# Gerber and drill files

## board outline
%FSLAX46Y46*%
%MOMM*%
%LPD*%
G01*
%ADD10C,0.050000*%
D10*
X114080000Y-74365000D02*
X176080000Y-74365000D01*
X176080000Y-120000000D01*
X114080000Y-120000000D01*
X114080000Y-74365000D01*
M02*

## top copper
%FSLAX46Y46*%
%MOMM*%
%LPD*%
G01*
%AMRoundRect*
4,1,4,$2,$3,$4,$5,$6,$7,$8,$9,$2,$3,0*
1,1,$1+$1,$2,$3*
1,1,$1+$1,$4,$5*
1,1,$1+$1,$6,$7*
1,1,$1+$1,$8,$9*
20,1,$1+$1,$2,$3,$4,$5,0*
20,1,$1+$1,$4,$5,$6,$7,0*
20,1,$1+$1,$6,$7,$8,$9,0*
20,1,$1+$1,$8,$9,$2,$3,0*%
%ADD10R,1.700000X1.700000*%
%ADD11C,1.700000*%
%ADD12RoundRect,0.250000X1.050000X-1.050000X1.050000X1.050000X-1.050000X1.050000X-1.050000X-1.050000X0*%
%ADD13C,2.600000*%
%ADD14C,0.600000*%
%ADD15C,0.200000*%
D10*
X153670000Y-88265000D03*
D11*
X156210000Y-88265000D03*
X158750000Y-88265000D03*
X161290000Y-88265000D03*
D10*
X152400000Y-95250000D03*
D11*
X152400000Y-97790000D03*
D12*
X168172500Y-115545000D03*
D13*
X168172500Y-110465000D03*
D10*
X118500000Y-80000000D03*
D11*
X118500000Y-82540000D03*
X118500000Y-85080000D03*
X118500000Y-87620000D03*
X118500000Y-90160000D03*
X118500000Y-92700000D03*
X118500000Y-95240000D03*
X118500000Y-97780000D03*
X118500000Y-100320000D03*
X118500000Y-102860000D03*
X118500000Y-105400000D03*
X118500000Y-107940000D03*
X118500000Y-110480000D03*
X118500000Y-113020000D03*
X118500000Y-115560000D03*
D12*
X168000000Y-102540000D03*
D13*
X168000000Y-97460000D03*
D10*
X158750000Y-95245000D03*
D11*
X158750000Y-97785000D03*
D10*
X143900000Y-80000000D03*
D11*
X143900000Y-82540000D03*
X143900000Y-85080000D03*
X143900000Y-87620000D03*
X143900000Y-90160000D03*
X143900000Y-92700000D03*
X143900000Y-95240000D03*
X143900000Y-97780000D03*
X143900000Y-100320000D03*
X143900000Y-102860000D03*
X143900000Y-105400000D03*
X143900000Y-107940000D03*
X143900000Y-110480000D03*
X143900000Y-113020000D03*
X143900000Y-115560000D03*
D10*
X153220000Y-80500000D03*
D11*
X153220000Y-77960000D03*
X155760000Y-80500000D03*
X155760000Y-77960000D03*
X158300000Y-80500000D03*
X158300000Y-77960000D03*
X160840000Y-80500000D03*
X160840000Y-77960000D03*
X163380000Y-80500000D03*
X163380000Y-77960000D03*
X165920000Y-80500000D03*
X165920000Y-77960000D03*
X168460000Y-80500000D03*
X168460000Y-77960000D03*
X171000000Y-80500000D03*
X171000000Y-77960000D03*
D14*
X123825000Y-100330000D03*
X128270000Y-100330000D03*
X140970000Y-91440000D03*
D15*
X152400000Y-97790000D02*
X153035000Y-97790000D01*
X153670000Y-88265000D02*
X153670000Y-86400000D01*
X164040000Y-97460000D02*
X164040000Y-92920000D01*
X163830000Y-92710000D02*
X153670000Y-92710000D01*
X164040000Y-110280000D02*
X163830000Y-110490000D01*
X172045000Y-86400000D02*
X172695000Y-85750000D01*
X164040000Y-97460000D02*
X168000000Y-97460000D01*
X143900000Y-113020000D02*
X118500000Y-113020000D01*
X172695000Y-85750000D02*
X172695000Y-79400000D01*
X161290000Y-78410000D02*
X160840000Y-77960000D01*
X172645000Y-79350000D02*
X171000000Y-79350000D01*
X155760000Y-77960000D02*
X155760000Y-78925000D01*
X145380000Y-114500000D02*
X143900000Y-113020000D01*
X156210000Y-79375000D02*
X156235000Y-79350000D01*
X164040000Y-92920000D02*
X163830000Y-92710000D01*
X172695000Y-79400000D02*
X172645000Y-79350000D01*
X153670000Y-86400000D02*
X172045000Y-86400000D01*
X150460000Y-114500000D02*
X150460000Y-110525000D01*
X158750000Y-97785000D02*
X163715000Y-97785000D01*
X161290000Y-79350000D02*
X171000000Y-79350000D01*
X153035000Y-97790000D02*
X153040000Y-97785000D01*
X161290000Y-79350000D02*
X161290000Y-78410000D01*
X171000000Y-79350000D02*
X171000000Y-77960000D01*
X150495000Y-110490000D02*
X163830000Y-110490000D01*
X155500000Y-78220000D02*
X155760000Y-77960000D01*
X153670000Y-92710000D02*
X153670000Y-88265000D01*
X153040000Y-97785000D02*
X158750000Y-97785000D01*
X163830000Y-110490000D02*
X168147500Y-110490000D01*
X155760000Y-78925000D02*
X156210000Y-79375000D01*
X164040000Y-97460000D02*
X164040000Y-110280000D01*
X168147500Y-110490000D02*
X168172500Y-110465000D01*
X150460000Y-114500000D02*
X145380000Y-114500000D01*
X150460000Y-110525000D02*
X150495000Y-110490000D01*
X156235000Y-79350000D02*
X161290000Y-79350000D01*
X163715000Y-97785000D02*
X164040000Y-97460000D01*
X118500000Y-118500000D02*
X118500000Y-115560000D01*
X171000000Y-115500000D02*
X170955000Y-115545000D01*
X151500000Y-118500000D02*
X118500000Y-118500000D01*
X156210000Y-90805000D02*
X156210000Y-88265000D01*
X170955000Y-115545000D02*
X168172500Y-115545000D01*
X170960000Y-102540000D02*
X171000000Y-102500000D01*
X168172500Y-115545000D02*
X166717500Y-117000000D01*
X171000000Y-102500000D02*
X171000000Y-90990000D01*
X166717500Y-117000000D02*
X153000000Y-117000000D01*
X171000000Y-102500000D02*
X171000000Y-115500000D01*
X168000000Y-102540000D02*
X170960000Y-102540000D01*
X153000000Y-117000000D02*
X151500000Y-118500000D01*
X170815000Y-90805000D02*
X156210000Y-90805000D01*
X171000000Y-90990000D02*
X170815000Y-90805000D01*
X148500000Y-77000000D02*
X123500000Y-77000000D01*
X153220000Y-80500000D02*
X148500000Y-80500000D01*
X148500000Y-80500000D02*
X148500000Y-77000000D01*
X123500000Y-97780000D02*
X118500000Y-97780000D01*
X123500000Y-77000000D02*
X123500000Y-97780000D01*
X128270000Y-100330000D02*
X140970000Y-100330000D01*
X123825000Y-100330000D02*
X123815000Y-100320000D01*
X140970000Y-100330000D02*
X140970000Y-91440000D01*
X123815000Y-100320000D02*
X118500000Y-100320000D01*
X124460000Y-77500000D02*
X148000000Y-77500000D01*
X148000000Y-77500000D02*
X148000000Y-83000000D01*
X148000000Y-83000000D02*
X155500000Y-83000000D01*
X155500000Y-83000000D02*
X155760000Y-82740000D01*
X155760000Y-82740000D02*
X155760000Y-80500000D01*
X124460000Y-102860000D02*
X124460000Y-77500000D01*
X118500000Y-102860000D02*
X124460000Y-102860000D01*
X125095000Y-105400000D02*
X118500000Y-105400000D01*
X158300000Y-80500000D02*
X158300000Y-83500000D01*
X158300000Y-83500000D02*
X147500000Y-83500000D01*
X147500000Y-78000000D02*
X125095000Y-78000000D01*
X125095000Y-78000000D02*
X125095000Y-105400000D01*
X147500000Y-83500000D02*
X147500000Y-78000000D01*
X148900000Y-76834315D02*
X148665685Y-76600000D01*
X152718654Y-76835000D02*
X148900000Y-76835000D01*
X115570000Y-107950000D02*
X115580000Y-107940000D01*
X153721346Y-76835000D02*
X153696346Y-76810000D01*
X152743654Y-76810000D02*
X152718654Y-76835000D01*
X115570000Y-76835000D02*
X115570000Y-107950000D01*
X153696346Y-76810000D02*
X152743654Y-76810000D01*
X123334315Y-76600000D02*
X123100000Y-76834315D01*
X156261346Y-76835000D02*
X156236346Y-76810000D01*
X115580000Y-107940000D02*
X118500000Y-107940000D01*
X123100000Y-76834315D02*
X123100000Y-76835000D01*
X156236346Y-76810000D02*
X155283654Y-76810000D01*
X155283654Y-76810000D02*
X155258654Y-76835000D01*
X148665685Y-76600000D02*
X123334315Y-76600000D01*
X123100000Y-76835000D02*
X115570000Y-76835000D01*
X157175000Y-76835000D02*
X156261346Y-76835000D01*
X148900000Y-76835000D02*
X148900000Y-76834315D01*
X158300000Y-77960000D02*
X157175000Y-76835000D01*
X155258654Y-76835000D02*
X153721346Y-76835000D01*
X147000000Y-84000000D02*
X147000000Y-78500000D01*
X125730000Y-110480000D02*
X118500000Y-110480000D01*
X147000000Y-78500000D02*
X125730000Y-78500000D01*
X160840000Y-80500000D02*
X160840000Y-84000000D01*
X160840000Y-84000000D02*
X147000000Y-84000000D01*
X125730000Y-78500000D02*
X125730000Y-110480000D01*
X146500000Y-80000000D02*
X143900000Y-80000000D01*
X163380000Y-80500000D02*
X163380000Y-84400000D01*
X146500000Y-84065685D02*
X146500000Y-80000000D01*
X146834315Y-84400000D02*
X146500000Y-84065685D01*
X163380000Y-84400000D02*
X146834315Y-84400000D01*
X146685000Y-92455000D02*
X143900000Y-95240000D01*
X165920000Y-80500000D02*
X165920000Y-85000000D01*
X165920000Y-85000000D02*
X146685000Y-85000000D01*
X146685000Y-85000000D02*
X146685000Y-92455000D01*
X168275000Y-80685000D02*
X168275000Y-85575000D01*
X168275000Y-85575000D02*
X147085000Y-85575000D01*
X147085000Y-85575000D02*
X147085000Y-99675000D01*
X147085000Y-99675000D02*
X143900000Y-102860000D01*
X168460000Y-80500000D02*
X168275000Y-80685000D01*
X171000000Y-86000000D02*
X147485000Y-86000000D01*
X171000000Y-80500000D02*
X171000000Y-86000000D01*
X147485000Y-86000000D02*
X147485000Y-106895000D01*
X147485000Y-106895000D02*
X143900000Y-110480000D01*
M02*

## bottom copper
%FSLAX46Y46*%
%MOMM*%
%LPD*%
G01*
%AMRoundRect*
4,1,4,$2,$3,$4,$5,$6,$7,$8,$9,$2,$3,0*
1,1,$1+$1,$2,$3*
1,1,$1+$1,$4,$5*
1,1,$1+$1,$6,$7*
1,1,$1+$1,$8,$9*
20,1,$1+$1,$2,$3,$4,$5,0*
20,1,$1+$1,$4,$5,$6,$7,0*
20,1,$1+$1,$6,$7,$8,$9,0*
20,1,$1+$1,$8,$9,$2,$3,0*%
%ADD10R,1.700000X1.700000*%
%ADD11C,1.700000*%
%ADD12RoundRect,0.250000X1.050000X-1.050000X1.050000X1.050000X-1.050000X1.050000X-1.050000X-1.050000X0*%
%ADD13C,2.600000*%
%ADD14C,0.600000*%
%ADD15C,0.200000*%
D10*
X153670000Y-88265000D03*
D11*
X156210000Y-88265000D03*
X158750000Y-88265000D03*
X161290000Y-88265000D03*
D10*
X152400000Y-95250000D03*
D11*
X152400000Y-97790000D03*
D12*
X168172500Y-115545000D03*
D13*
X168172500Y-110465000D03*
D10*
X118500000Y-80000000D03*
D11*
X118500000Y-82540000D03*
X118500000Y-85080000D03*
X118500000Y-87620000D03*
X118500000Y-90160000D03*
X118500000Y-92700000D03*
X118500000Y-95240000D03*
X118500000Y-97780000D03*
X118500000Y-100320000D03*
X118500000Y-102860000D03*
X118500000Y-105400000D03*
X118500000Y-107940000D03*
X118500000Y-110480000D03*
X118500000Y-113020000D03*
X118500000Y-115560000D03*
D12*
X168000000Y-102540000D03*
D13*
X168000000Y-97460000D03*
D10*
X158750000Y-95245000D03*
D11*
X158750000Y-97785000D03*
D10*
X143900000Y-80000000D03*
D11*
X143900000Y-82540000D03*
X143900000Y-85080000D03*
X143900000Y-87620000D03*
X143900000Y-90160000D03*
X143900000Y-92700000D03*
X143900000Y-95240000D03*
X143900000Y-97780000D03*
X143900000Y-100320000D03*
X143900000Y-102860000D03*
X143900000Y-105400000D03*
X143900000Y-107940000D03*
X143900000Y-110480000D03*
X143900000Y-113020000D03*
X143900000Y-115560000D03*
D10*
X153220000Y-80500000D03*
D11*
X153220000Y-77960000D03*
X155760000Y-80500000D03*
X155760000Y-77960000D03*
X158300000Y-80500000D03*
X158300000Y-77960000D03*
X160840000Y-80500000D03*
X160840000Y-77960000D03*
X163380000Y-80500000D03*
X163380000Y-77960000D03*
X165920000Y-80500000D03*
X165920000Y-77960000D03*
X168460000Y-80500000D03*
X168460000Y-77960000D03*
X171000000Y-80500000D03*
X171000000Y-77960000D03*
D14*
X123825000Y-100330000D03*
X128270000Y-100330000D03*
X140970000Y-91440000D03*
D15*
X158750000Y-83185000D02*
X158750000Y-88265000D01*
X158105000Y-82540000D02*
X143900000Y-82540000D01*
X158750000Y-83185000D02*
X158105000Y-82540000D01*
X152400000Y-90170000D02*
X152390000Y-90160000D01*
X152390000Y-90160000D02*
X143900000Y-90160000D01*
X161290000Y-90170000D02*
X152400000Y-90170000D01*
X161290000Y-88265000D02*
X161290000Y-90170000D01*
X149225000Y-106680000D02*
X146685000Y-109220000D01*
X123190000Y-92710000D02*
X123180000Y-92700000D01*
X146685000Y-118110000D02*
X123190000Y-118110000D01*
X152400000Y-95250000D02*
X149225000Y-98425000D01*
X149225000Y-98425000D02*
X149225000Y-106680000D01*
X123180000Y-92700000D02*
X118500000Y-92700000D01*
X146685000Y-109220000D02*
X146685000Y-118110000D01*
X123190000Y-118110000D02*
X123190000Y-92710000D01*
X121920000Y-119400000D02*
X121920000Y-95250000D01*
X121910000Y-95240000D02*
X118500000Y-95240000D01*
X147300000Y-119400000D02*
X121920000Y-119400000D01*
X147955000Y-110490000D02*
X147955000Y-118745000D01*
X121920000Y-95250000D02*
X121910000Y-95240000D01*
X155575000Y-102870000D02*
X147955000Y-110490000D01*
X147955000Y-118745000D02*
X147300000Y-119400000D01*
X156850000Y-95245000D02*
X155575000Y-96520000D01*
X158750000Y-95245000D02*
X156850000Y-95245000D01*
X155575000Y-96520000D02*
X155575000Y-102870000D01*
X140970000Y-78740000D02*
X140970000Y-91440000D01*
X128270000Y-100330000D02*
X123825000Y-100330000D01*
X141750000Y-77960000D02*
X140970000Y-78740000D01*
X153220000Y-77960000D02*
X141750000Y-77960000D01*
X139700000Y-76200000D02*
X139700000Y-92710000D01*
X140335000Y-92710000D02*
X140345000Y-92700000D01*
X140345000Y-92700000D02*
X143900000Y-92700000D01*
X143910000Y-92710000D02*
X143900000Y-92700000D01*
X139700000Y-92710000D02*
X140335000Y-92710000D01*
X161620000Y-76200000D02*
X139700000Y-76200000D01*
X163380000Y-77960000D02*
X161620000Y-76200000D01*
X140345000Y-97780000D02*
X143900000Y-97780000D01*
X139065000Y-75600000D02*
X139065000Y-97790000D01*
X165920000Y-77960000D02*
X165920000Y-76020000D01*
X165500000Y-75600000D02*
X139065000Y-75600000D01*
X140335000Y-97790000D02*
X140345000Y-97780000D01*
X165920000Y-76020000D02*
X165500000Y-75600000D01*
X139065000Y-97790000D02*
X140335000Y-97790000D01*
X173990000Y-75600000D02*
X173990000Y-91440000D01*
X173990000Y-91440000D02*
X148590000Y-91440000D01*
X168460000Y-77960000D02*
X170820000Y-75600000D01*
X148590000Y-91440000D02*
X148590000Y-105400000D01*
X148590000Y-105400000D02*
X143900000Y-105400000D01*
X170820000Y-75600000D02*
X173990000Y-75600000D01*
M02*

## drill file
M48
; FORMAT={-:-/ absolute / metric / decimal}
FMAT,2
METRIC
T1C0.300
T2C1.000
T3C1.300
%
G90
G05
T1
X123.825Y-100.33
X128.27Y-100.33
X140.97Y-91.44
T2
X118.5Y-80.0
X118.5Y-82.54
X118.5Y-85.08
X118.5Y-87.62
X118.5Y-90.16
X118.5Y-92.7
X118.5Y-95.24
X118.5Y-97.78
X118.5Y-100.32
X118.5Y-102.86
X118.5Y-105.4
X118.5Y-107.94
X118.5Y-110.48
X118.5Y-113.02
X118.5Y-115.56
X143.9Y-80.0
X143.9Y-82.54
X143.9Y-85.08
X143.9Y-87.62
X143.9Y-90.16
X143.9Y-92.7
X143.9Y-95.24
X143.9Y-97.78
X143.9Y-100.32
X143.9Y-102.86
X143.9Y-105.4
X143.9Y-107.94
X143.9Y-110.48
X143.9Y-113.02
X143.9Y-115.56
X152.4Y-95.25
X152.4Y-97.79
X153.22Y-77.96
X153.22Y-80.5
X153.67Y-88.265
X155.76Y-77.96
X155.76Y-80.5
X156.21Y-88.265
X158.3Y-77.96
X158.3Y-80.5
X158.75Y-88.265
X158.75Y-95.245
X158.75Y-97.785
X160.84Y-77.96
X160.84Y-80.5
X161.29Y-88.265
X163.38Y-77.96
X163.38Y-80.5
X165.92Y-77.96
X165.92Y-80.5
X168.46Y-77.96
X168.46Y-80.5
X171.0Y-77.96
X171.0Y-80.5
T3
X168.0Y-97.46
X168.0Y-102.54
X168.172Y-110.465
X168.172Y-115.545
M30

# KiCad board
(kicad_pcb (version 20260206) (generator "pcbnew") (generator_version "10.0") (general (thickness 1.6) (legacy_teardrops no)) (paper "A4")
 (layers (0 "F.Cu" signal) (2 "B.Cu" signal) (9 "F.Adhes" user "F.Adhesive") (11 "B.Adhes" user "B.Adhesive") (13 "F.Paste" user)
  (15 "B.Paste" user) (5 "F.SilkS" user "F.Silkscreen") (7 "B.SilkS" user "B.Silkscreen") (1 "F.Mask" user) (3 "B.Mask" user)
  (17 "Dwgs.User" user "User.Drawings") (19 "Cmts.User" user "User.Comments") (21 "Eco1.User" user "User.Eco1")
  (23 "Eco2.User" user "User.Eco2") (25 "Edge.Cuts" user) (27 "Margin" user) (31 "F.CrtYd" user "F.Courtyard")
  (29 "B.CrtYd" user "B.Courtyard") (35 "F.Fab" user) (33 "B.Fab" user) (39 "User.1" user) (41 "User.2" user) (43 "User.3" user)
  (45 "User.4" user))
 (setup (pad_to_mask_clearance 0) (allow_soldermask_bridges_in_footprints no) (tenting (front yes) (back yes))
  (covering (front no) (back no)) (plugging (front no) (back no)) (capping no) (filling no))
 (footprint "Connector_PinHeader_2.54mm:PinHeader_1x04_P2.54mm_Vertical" (layer "F.Cu") (at 153.67 88.265 90)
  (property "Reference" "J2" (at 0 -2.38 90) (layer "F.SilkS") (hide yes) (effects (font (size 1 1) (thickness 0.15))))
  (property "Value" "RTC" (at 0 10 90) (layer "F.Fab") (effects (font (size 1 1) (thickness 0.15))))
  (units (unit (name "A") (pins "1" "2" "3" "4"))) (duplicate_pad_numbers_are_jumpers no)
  (pad "1" thru_hole rect (at 0 0 90) (size 1.7 1.7) (drill 1) (layers "*.Cu" "*.Mask") (remove_unused_layers no) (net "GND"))
  (pad "2" thru_hole circle (at 0 2.54 90) (size 1.7 1.7) (drill 1) (layers "*.Cu" "*.Mask") (remove_unused_layers no) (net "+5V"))
  (pad "3" thru_hole circle (at 0 5.08 90) (size 1.7 1.7) (drill 1) (layers "*.Cu" "*.Mask") (remove_unused_layers no) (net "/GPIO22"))
  (pad "4" thru_hole circle (at 0 7.62 90) (size 1.7 1.7) (drill 1) (layers "*.Cu" "*.Mask") (remove_unused_layers no) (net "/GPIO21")))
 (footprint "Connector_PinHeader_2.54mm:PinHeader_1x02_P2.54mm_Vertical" (layer "F.Cu") (at 152.4 95.25)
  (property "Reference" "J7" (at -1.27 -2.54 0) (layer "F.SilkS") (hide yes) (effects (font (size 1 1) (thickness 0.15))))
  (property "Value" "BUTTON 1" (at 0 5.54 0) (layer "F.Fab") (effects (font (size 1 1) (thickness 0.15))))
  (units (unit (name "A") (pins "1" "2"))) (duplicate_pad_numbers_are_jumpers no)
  (pad "1" thru_hole rect (at 0 0) (size 1.7 1.7) (drill 1) (layers "*.Cu" "*.Mask") (remove_unused_layers no) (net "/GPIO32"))
  (pad "2" thru_hole circle (at 0 2.54) (size 1.7 1.7) (drill 1) (layers "*.Cu" "*.Mask") (remove_unused_layers no) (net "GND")))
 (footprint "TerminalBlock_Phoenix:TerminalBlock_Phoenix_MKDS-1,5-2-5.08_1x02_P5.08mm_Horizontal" (layer "F.Cu") (at 168.1725 115.545 90)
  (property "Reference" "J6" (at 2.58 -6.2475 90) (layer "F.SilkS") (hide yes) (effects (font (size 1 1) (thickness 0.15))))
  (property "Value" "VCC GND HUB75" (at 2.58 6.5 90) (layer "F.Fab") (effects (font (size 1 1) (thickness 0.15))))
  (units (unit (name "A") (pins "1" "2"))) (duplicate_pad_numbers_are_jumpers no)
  (pad "1" thru_hole roundrect (at 0 0 90) (size 2.6 2.6) (drill 1.3) (layers "*.Cu" "*.Mask") (remove_unused_layers no)
   (roundrect_rratio 0.096154) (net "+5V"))
  (pad "2" thru_hole circle (at 5.08 0 90) (size 2.6 2.6) (drill 1.3) (layers "*.Cu" "*.Mask") (remove_unused_layers no) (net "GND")))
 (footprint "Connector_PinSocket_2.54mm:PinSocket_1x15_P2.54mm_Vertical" (layer "F.Cu") (at 118.5 80)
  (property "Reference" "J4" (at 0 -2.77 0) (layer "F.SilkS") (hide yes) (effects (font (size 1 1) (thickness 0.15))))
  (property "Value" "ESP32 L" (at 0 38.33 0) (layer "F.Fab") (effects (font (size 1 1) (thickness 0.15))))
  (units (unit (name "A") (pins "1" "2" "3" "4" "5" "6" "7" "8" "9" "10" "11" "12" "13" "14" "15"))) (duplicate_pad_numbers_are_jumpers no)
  (pad "1" thru_hole rect (at 0 0) (size 1.7 1.7) (drill 1) (layers "*.Cu" "*.Mask") (remove_unused_layers no)
   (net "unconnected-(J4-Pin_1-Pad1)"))
  (pad "2" thru_hole circle (at 0 2.54) (size 1.7 1.7) (drill 1) (layers "*.Cu" "*.Mask") (remove_unused_layers no)
   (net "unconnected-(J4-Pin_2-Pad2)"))
  (pad "3" thru_hole circle (at 0 5.08) (size 1.7 1.7) (drill 1) (layers "*.Cu" "*.Mask") (remove_unused_layers no)
   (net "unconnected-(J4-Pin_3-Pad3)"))
  (pad "4" thru_hole circle (at 0 7.62) (size 1.7 1.7) (drill 1) (layers "*.Cu" "*.Mask") (remove_unused_layers no)
   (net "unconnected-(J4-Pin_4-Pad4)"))
  (pad "5" thru_hole circle (at 0 10.16) (size 1.7 1.7) (drill 1) (layers "*.Cu" "*.Mask") (remove_unused_layers no)
   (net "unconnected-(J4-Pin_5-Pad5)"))
  (pad "6" thru_hole circle (at 0 12.7) (size 1.7 1.7) (drill 1) (layers "*.Cu" "*.Mask") (remove_unused_layers no) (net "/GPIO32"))
  (pad "7" thru_hole circle (at 0 15.24) (size 1.7 1.7) (drill 1) (layers "*.Cu" "*.Mask") (remove_unused_layers no) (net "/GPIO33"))
  (pad "8" thru_hole circle (at 0 17.78) (size 1.7 1.7) (drill 1) (layers "*.Cu" "*.Mask") (remove_unused_layers no) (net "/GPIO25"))
  (pad "9" thru_hole circle (at 0 20.32) (size 1.7 1.7) (drill 1) (layers "*.Cu" "*.Mask") (remove_unused_layers no) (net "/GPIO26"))
  (pad "10" thru_hole circle (at 0 22.86) (size 1.7 1.7) (drill 1) (layers "*.Cu" "*.Mask") (remove_unused_layers no) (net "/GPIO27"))
  (pad "11" thru_hole circle (at 0 25.4) (size 1.7 1.7) (drill 1) (layers "*.Cu" "*.Mask") (remove_unused_layers no) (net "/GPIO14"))
  (pad "12" thru_hole circle (at 0 27.94) (size 1.7 1.7) (drill 1) (layers "*.Cu" "*.Mask") (remove_unused_layers no) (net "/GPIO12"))
  (pad "13" thru_hole circle (at 0 30.48) (size 1.7 1.7) (drill 1) (layers "*.Cu" "*.Mask") (remove_unused_layers no) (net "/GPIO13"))
  (pad "14" thru_hole circle (at 0 33.02) (size 1.7 1.7) (drill 1) (layers "*.Cu" "*.Mask") (remove_unused_layers no) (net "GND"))
  (pad "15" thru_hole circle (at 0 35.56) (size 1.7 1.7) (drill 1) (layers "*.Cu" "*.Mask") (remove_unused_layers no) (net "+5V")))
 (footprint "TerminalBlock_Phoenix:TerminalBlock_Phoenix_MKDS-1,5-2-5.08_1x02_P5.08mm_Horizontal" (layer "F.Cu") (at 168 102.54 90)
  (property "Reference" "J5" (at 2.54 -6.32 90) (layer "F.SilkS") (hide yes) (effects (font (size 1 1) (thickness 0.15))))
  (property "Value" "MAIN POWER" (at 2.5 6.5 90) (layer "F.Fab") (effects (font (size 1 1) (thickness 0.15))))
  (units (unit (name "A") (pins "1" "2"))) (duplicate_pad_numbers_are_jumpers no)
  (pad "1" thru_hole roundrect (at 0 0 90) (size 2.6 2.6) (drill 1.3) (layers "*.Cu" "*.Mask") (remove_unused_layers no)
   (roundrect_rratio 0.096154) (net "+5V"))
  (pad "2" thru_hole circle (at 5.08 0 90) (size 2.6 2.6) (drill 1.3) (layers "*.Cu" "*.Mask") (remove_unused_layers no) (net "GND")))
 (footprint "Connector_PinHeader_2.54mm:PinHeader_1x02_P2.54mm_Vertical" (layer "F.Cu") (at 158.75 95.245)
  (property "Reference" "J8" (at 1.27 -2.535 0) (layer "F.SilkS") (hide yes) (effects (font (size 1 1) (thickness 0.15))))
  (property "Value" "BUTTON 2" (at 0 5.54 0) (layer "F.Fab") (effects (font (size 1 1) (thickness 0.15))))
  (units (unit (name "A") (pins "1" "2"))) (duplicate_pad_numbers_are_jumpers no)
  (pad "1" thru_hole rect (at 0 0) (size 1.7 1.7) (drill 1) (layers "*.Cu" "*.Mask") (remove_unused_layers no) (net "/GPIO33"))
  (pad "2" thru_hole circle (at 0 2.54) (size 1.7 1.7) (drill 1) (layers "*.Cu" "*.Mask") (remove_unused_layers no) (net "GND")))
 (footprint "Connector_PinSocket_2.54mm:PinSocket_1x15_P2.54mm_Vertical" (layer "F.Cu") (at 143.9 80)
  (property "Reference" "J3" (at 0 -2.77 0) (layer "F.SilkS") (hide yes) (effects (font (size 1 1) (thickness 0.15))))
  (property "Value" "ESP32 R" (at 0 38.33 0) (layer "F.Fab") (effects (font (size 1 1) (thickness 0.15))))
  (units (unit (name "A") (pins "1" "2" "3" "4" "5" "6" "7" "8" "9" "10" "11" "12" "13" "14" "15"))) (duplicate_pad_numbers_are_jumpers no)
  (pad "1" thru_hole rect (at 0 0) (size 1.7 1.7) (drill 1) (layers "*.Cu" "*.Mask") (remove_unused_layers no) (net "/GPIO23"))
  (pad "2" thru_hole circle (at 0 2.54) (size 1.7 1.7) (drill 1) (layers "*.Cu" "*.Mask") (remove_unused_layers no) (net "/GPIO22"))
  (pad "3" thru_hole circle (at 0 5.08) (size 1.7 1.7) (drill 1) (layers "*.Cu" "*.Mask") (remove_unused_layers no)
   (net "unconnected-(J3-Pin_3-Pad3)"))
  (pad "4" thru_hole circle (at 0 7.62) (size 1.7 1.7) (drill 1) (layers "*.Cu" "*.Mask") (remove_unused_layers no)
   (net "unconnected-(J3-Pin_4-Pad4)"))
  (pad "5" thru_hole circle (at 0 10.16) (size 1.7 1.7) (drill 1) (layers "*.Cu" "*.Mask") (remove_unused_layers no) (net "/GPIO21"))
  (pad "6" thru_hole circle (at 0 12.7) (size 1.7 1.7) (drill 1) (layers "*.Cu" "*.Mask") (remove_unused_layers no) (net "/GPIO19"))
  (pad "7" thru_hole circle (at 0 15.24) (size 1.7 1.7) (drill 1) (layers "*.Cu" "*.Mask") (remove_unused_layers no) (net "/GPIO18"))
  (pad "8" thru_hole circle (at 0 17.78) (size 1.7 1.7) (drill 1) (layers "*.Cu" "*.Mask") (remove_unused_layers no) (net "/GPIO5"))
  (pad "9" thru_hole circle (at 0 20.32) (size 1.7 1.7) (drill 1) (layers "*.Cu" "*.Mask") (remove_unused_layers no)
   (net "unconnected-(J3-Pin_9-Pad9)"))
  (pad "10" thru_hole circle (at 0 22.86) (size 1.7 1.7) (drill 1) (layers "*.Cu" "*.Mask") (remove_unused_layers no) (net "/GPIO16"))
  (pad "11" thru_hole circle (at 0 25.4) (size 1.7 1.7) (drill 1) (layers "*.Cu" "*.Mask") (remove_unused_layers no) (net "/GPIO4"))
  (pad "12" thru_hole circle (at 0 27.94) (size 1.7 1.7) (drill 1) (layers "*.Cu" "*.Mask") (remove_unused_layers no)
   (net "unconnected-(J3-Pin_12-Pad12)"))
  (pad "13" thru_hole circle (at 0 30.48) (size 1.7 1.7) (drill 1) (layers "*.Cu" "*.Mask") (remove_unused_layers no) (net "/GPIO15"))
  (pad "14" thru_hole circle (at 0 33.02) (size 1.7 1.7) (drill 1) (layers "*.Cu" "*.Mask") (remove_unused_layers no) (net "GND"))
  (pad "15" thru_hole circle (at 0 35.56) (size 1.7 1.7) (drill 1) (layers "*.Cu" "*.Mask") (remove_unused_layers no)
   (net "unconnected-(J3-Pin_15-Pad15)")))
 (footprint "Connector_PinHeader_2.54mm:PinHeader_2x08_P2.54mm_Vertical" (layer "F.Cu") (at 153.22 80.5 90)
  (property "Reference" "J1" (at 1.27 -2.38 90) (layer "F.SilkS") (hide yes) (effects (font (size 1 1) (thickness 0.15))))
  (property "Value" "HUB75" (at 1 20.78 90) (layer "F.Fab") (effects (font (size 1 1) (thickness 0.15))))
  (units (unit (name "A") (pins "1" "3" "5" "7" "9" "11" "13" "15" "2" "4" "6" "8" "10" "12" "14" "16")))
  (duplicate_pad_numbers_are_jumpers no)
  (pad "1" thru_hole rect (at 0 0 90) (size 1.7 1.7) (drill 1) (layers "*.Cu" "*.Mask") (remove_unused_layers no) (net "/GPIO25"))
  (pad "2" thru_hole circle (at 2.54 0 90) (size 1.7 1.7) (drill 1) (layers "*.Cu" "*.Mask") (remove_unused_layers no) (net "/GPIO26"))
  (pad "3" thru_hole circle (at 0 2.54 90) (size 1.7 1.7) (drill 1) (layers "*.Cu" "*.Mask") (remove_unused_layers no) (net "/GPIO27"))
  (pad "4" thru_hole circle (at 2.54 2.54 90) (size 1.7 1.7) (drill 1) (layers "*.Cu" "*.Mask") (remove_unused_layers no) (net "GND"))
  (pad "5" thru_hole circle (at 0 5.08 90) (size 1.7 1.7) (drill 1) (layers "*.Cu" "*.Mask") (remove_unused_layers no) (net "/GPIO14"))
  (pad "6" thru_hole circle (at 2.54 5.08 90) (size 1.7 1.7) (drill 1) (layers "*.Cu" "*.Mask") (remove_unused_layers no) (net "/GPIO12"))
  (pad "7" thru_hole circle (at 0 7.62 90) (size 1.7 1.7) (drill 1) (layers "*.Cu" "*.Mask") (remove_unused_layers no) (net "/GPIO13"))
  (pad "8" thru_hole circle (at 2.54 7.62 90) (size 1.7 1.7) (drill 1) (layers "*.Cu" "*.Mask") (remove_unused_layers no) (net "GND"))
  (pad "9" thru_hole circle (at 0 10.16 90) (size 1.7 1.7) (drill 1) (layers "*.Cu" "*.Mask") (remove_unused_layers no) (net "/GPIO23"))
  (pad "10" thru_hole circle (at 2.54 10.16 90) (size 1.7 1.7) (drill 1) (layers "*.Cu" "*.Mask") (remove_unused_layers no) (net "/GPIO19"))
  (pad "11" thru_hole circle (at 0 12.7 90) (size 1.7 1.7) (drill 1) (layers "*.Cu" "*.Mask") (remove_unused_layers no) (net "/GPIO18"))
  (pad "12" thru_hole circle (at 2.54 12.7 90) (size 1.7 1.7) (drill 1) (layers "*.Cu" "*.Mask") (remove_unused_layers no) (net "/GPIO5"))
  (pad "13" thru_hole circle (at 0 15.24 90) (size 1.7 1.7) (drill 1) (layers "*.Cu" "*.Mask") (remove_unused_layers no) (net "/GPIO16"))
  (pad "14" thru_hole circle (at 2.54 15.24 90) (size 1.7 1.7) (drill 1) (layers "*.Cu" "*.Mask") (remove_unused_layers no) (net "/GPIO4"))
  (pad "15" thru_hole circle (at 0 17.78 90) (size 1.7 1.7) (drill 1) (layers "*.Cu" "*.Mask") (remove_unused_layers no) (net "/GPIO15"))
  (pad "16" thru_hole circle (at 2.54 17.78 90) (size 1.7 1.7) (drill 1) (layers "*.Cu" "*.Mask") (remove_unused_layers no) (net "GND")))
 (gr_rect (start 114.08 74.365) (end 176.08 120) (stroke (width 0.05) (type solid)) (fill no) (layer "Edge.Cuts"))
 (segment (start 152.4 97.79) (end 153.035 97.79) (width 0.2) (layer "F.Cu") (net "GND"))
 (segment (start 153.67 88.265) (end 153.67 86.4) (width 0.2) (layer "F.Cu") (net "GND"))
 (segment (start 164.04 97.46) (end 164.04 92.92) (width 0.2) (layer "F.Cu") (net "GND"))
 (segment (start 163.83 92.71) (end 153.67 92.71) (width 0.2) (layer "F.Cu") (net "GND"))
 (segment (start 164.04 110.28) (end 163.83 110.49) (width 0.2) (layer "F.Cu") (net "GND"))
 (segment (start 172.045 86.4) (end 172.695 85.75) (width 0.2) (layer "F.Cu") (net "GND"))
 (segment (start 164.04 97.46) (end 168 97.46) (width 0.2) (layer "F.Cu") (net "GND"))
 (segment (start 143.9 113.02) (end 118.5 113.02) (width 0.2) (layer "F.Cu") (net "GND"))
 (segment (start 172.695 85.75) (end 172.695 79.4) (width 0.2) (layer "F.Cu") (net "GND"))
 (segment (start 161.29 78.41) (end 160.84 77.96) (width 0.2) (layer "F.Cu") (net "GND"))
 (segment (start 172.645 79.35) (end 171 79.35) (width 0.2) (layer "F.Cu") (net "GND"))
 (segment (start 155.76 77.96) (end 155.76 78.925) (width 0.2) (layer "F.Cu") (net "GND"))
 (segment (start 145.38 114.5) (end 143.9 113.02) (width 0.2) (layer "F.Cu") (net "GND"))
 (segment (start 156.21 79.375) (end 156.235 79.35) (width 0.2) (layer "F.Cu") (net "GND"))
 (segment (start 164.04 92.92) (end 163.83 92.71) (width 0.2) (layer "F.Cu") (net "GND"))
 (segment (start 172.695 79.4) (end 172.645 79.35) (width 0.2) (layer "F.Cu") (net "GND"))
 (segment (start 153.67 86.4) (end 172.045 86.4) (width 0.2) (layer "F.Cu") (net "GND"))
 (segment (start 150.46 114.5) (end 150.46 110.525) (width 0.2) (layer "F.Cu") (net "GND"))
 (segment (start 158.75 97.785) (end 163.715 97.785) (width 0.2) (layer "F.Cu") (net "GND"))
 (segment (start 161.29 79.35) (end 171 79.35) (width 0.2) (layer "F.Cu") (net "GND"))
 (segment (start 153.035 97.79) (end 153.04 97.785) (width 0.2) (layer "F.Cu") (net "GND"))
 (segment (start 161.29 79.35) (end 161.29 78.41) (width 0.2) (layer "F.Cu") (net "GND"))
 (segment (start 171 79.35) (end 171 77.96) (width 0.2) (layer "F.Cu") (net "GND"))
 (segment (start 150.495 110.49) (end 163.83 110.49) (width 0.2) (layer "F.Cu") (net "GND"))
 (segment (start 155.5 78.22) (end 155.76 77.96) (width 0.2) (layer "F.Cu") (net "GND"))
 (segment (start 153.67 92.71) (end 153.67 88.265) (width 0.2) (layer "F.Cu") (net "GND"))
 (segment (start 153.04 97.785) (end 158.75 97.785) (width 0.2) (layer "F.Cu") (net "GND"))
 (segment (start 163.83 110.49) (end 168.1475 110.49) (width 0.2) (layer "F.Cu") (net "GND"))
 (segment (start 155.76 78.925) (end 156.21 79.375) (width 0.2) (layer "F.Cu") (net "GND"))
 (segment (start 164.04 97.46) (end 164.04 110.28) (width 0.2) (layer "F.Cu") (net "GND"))
 (segment (start 168.1475 110.49) (end 168.1725 110.465) (width 0.2) (layer "F.Cu") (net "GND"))
 (segment (start 150.46 114.5) (end 145.38 114.5) (width 0.2) (layer "F.Cu") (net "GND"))
 (segment (start 150.46 110.525) (end 150.495 110.49) (width 0.2) (layer "F.Cu") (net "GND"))
 (segment (start 156.235 79.35) (end 161.29 79.35) (width 0.2) (layer "F.Cu") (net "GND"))
 (segment (start 163.715 97.785) (end 164.04 97.46) (width 0.2) (layer "F.Cu") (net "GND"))
 (segment (start 118.5 118.5) (end 118.5 115.56) (width 0.2) (layer "F.Cu") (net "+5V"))
 (segment (start 171 115.5) (end 170.955 115.545) (width 0.2) (layer "F.Cu") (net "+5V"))
 (segment (start 151.5 118.5) (end 118.5 118.5) (width 0.2) (layer "F.Cu") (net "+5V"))
 (segment (start 156.21 90.805) (end 156.21 88.265) (width 0.2) (layer "F.Cu") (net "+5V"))
 (segment (start 170.955 115.545) (end 168.1725 115.545) (width 0.2) (layer "F.Cu") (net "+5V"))
 (segment (start 170.96 102.54) (end 171 102.5) (width 0.2) (layer "F.Cu") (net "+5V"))
 (segment (start 168.1725 115.545) (end 166.7175 117) (width 0.2) (layer "F.Cu") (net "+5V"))
 (segment (start 171 102.5) (end 171 90.99) (width 0.2) (layer "F.Cu") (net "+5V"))
 (segment (start 166.7175 117) (end 153 117) (width 0.2) (layer "F.Cu") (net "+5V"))
 (segment (start 171 102.5) (end 171 115.5) (width 0.2) (layer "F.Cu") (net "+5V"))
 (segment (start 168 102.54) (end 170.96 102.54) (width 0.2) (layer "F.Cu") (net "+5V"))
 (segment (start 153 117) (end 151.5 118.5) (width 0.2) (layer "F.Cu") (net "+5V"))
 (segment (start 170.815 90.805) (end 156.21 90.805) (width 0.2) (layer "F.Cu") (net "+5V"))
 (segment (start 171 90.99) (end 170.815 90.805) (width 0.2) (layer "F.Cu") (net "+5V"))
 (segment (start 158.75 83.185) (end 158.75 88.265) (width 0.2) (layer "B.Cu") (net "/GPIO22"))
 (segment (start 158.105 82.54) (end 143.9 82.54) (width 0.2) (layer "B.Cu") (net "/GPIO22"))
 (segment (start 158.75 83.185) (end 158.105 82.54) (width 0.2) (layer "B.Cu") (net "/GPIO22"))
 (segment (start 152.4 90.17) (end 152.39 90.16) (width 0.2) (layer "B.Cu") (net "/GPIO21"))
 (segment (start 152.39 90.16) (end 143.9 90.16) (width 0.2) (layer "B.Cu") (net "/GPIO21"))
 (segment (start 161.29 90.17) (end 152.4 90.17) (width 0.2) (layer "B.Cu") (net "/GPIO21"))
 (segment (start 161.29 88.265) (end 161.29 90.17) (width 0.2) (layer "B.Cu") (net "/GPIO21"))
 (segment (start 149.225 106.68) (end 146.685 109.22) (width 0.2) (layer "B.Cu") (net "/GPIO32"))
 (segment (start 123.19 92.71) (end 123.18 92.7) (width 0.2) (layer "B.Cu") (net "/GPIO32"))
 (segment (start 146.685 118.11) (end 123.19 118.11) (width 0.2) (layer "B.Cu") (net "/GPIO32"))
 (segment (start 152.4 95.25) (end 149.225 98.425) (width 0.2) (layer "B.Cu") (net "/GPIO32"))
 (segment (start 149.225 98.425) (end 149.225 106.68) (width 0.2) (layer "B.Cu") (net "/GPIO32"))
 (segment (start 123.18 92.7) (end 118.5 92.7) (width 0.2) (layer "B.Cu") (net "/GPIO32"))
 (segment (start 146.685 109.22) (end 146.685 118.11) (width 0.2) (layer "B.Cu") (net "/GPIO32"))
 (segment (start 123.19 118.11) (end 123.19 92.71) (width 0.2) (layer "B.Cu") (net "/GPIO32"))
 (segment (start 121.92 119.4) (end 121.92 95.25) (width 0.2) (layer "B.Cu") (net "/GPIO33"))
 (segment (start 121.91 95.24) (end 118.5 95.24) (width 0.2) (layer "B.Cu") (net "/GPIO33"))
 (segment (start 147.3 119.4) (end 121.92 119.4) (width 0.2) (layer "B.Cu") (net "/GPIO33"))
 (segment (start 147.955 110.49) (end 147.955 118.745) (width 0.2) (layer "B.Cu") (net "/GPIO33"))
 (segment (start 121.92 95.25) (end 121.91 95.24) (width 0.2) (layer "B.Cu") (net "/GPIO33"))
 (segment (start 155.575 102.87) (end 147.955 110.49) (width 0.2) (layer "B.Cu") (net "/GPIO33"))
 (segment (start 147.955 118.745) (end 147.3 119.4) (width 0.2) (layer "B.Cu") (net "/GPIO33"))
 (segment (start 156.85 95.245) (end 155.575 96.52) (width 0.2) (layer "B.Cu") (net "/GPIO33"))
 (segment (start 158.75 95.245) (end 156.85 95.245) (width 0.2) (layer "B.Cu") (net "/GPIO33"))
 (segment (start 155.575 96.52) (end 155.575 102.87) (width 0.2) (layer "B.Cu") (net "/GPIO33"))
 (segment (start 148.5 77) (end 123.5 77) (width 0.2) (layer "F.Cu") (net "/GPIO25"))
 (segment (start 153.22 80.5) (end 148.5 80.5) (width 0.2) (layer "F.Cu") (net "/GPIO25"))
 (segment (start 148.5 80.5) (end 148.5 77) (width 0.2) (layer "F.Cu") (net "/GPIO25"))
 (segment (start 123.5 97.78) (end 118.5 97.78) (width 0.2) (layer "F.Cu") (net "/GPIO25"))
 (segment (start 123.5 77) (end 123.5 97.78) (width 0.2) (layer "F.Cu") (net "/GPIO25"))
 (segment (start 128.27 100.33) (end 140.97 100.33) (width 0.2) (layer "F.Cu") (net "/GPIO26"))
 (segment (start 123.825 100.33) (end 123.815 100.32) (width 0.2) (layer "F.Cu") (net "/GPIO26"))
 (segment (start 140.97 100.33) (end 140.97 91.44) (width 0.2) (layer "F.Cu") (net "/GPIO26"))
 (segment (start 123.815 100.32) (end 118.5 100.32) (width 0.2) (layer "F.Cu") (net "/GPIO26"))
 (via (at 123.825 100.33) (size 0.6) (drill 0.3) (layers "F.Cu" "B.Cu") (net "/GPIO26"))
 (via (at 128.27 100.33) (size 0.6) (drill 0.3) (layers "F.Cu" "B.Cu") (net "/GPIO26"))
 (via (at 140.97 91.44) (size 0.6) (drill 0.3) (layers "F.Cu" "B.Cu") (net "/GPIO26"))
 (segment (start 140.97 78.74) (end 140.97 91.44) (width 0.2) (layer "B.Cu") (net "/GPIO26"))
 (segment (start 128.27 100.33) (end 123.825 100.33) (width 0.2) (layer "B.Cu") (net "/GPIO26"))
 (segment (start 141.75 77.96) (end 140.97 78.74) (width 0.2) (layer "B.Cu") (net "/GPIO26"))
 (segment (start 153.22 77.96) (end 141.75 77.96) (width 0.2) (layer "B.Cu") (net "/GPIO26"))
 (segment (start 124.46 77.5) (end 148 77.5) (width 0.2) (layer "F.Cu") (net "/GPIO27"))
 (segment (start 148 77.5) (end 148 83) (width 0.2) (layer "F.Cu") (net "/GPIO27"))
 (segment (start 148 83) (end 155.5 83) (width 0.2) (layer "F.Cu") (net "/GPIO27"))
 (segment (start 155.5 83) (end 155.76 82.74) (width 0.2) (layer "F.Cu") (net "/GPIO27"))
 (segment (start 155.76 82.74) (end 155.76 80.5) (width 0.2) (layer "F.Cu") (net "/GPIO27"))
 (segment (start 124.46 102.86) (end 124.46 77.5) (width 0.2) (layer "F.Cu") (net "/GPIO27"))
 (segment (start 118.5 102.86) (end 124.46 102.86) (width 0.2) (layer "F.Cu") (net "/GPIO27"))
 (segment (start 125.095 105.4) (end 118.5 105.4) (width 0.2) (layer "F.Cu") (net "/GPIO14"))
 (segment (start 158.3 80.5) (end 158.3 83.5) (width 0.2) (layer "F.Cu") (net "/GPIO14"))
 (segment (start 158.3 83.5) (end 147.5 83.5) (width 0.2) (layer "F.Cu") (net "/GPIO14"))
 (segment (start 147.5 78) (end 125.095 78) (width 0.2) (layer "F.Cu") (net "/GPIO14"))
 (segment (start 125.095 78) (end 125.095 105.4) (width 0.2) (layer "F.Cu") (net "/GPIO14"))
 (segment (start 147.5 83.5) (end 147.5 78) (width 0.2) (layer "F.Cu") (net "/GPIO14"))
 (segment (start 148.9 76.834315) (end 148.665685 76.6) (width 0.2) (layer "F.Cu") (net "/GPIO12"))
 (segment (start 152.718654 76.835) (end 148.9 76.835) (width 0.2) (layer "F.Cu") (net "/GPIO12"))
 (segment (start 115.57 107.95) (end 115.58 107.94) (width 0.2) (layer "F.Cu") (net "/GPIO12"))
 (segment (start 153.721346 76.835) (end 153.696346 76.81) (width 0.2) (layer "F.Cu") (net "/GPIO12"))
 (segment (start 152.743654 76.81) (end 152.718654 76.835) (width 0.2) (layer "F.Cu") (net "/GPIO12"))
 (segment (start 115.57 76.835) (end 115.57 107.95) (width 0.2) (layer "F.Cu") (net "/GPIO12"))
 (segment (start 153.696346 76.81) (end 152.743654 76.81) (width 0.2) (layer "F.Cu") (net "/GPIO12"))
 (segment (start 123.334315 76.6) (end 123.1 76.834315) (width 0.2) (layer "F.Cu") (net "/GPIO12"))
 (segment (start 156.261346 76.835) (end 156.236346 76.81) (width 0.2) (layer "F.Cu") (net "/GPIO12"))
 (segment (start 115.58 107.94) (end 118.5 107.94) (width 0.2) (layer "F.Cu") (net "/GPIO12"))
 (segment (start 123.1 76.834315) (end 123.1 76.835) (width 0.2) (layer "F.Cu") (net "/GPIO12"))
 (segment (start 156.236346 76.81) (end 155.283654 76.81) (width 0.2) (layer "F.Cu") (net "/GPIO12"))
 (segment (start 155.283654 76.81) (end 155.258654 76.835) (width 0.2) (layer "F.Cu") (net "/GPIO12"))
 (segment (start 148.665685 76.6) (end 123.334315 76.6) (width 0.2) (layer "F.Cu") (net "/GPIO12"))
 (segment (start 123.1 76.835) (end 115.57 76.835) (width 0.2) (layer "F.Cu") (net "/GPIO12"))
 (segment (start 157.175 76.835) (end 156.261346 76.835) (width 0.2) (layer "F.Cu") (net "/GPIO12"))
 (segment (start 148.9 76.835) (end 148.9 76.834315) (width 0.2) (layer "F.Cu") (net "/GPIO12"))
 (segment (start 158.3 77.96) (end 157.175 76.835) (width 0.2) (layer "F.Cu") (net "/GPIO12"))
 (segment (start 155.258654 76.835) (end 153.721346 76.835) (width 0.2) (layer "F.Cu") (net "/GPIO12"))
 (segment (start 147 84) (end 147 78.5) (width 0.2) (layer "F.Cu") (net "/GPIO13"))
 (segment (start 125.73 110.48) (end 118.5 110.48) (width 0.2) (layer "F.Cu") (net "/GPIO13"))
 (segment (start 147 78.5) (end 125.73 78.5) (width 0.2) (layer "F.Cu") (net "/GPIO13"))
 (segment (start 160.84 80.5) (end 160.84 84) (width 0.2) (layer "F.Cu") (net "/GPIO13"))
 (segment (start 160.84 84) (end 147 84) (width 0.2) (layer "F.Cu") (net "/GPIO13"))
 (segment (start 125.73 78.5) (end 125.73 110.48) (width 0.2) (layer "F.Cu") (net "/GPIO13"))
 (segment (start 146.5 80) (end 143.9 80) (width 0.2) (layer "F.Cu") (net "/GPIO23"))
 (segment (start 163.38 80.5) (end 163.38 84.4) (width 0.2) (layer "F.Cu") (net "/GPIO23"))
 (segment (start 146.5 84.065685) (end 146.5 80) (width 0.2) (layer "F.Cu") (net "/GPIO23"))
 (segment (start 146.834315 84.4) (end 146.5 84.065685) (width 0.2) (layer "F.Cu") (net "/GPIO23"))
 (segment (start 163.38 84.4) (end 146.834315 84.4) (width 0.2) (layer "F.Cu") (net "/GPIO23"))
 (segment (start 139.7 76.2) (end 139.7 92.71) (width 0.2) (layer "B.Cu") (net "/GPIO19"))
 (segment (start 140.335 92.71) (end 140.345 92.7) (width 0.2) (layer "B.Cu") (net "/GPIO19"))
 (segment (start 140.345 92.7) (end 143.9 92.7) (width 0.2) (layer "B.Cu") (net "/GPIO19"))
 (segment (start 143.91 92.71) (end 143.9 92.7) (width 0.2) (layer "B.Cu") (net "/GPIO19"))
 (segment (start 139.7 92.71) (end 140.335 92.71) (width 0.2) (layer "B.Cu") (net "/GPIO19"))
 (segment (start 161.62 76.2) (end 139.7 76.2) (width 0.2) (layer "B.Cu") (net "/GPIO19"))
 (segment (start 163.38 77.96) (end 161.62 76.2) (width 0.2) (layer "B.Cu") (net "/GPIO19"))
 (segment (start 146.685 92.455) (end 143.9 95.24) (width 0.2) (layer "F.Cu") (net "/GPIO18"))
 (segment (start 165.92 80.5) (end 165.92 85) (width 0.2) (layer "F.Cu") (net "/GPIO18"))
 (segment (start 165.92 85) (end 146.685 85) (width 0.2) (layer "F.Cu") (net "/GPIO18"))
 (segment (start 146.685 85) (end 146.685 92.455) (width 0.2) (layer "F.Cu") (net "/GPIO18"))
 (segment (start 140.345 97.78) (end 143.9 97.78) (width 0.2) (layer "B.Cu") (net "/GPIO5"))
 (segment (start 139.065 75.6) (end 139.065 97.79) (width 0.2) (layer "B.Cu") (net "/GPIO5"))
 (segment (start 165.92 77.96) (end 165.92 76.02) (width 0.2) (layer "B.Cu") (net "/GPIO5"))
 (segment (start 165.5 75.6) (end 139.065 75.6) (width 0.2) (layer "B.Cu") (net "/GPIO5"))
 (segment (start 140.335 97.79) (end 140.345 97.78) (width 0.2) (layer "B.Cu") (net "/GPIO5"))
 (segment (start 165.92 76.02) (end 165.5 75.6) (width 0.2) (layer "B.Cu") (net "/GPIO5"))
 (segment (start 139.065 97.79) (end 140.335 97.79) (width 0.2) (layer "B.Cu") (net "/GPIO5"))
 (segment (start 168.275 80.685) (end 168.275 85.575) (width 0.2) (layer "F.Cu") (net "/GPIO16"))
 (segment (start 168.275 85.575) (end 147.085 85.575) (width 0.2) (layer "F.Cu") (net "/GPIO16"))
 (segment (start 147.085 85.575) (end 147.085 99.675) (width 0.2) (layer "F.Cu") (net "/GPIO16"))
 (segment (start 147.085 99.675) (end 143.9 102.86) (width 0.2) (layer "F.Cu") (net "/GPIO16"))
 (segment (start 168.46 80.5) (end 168.275 80.685) (width 0.2) (layer "F.Cu") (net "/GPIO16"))
 (segment (start 173.99 75.6) (end 173.99 91.44) (width 0.2) (layer "B.Cu") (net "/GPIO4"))
 (segment (start 173.99 91.44) (end 148.59 91.44) (width 0.2) (layer "B.Cu") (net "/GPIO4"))
 (segment (start 168.46 77.96) (end 170.82 75.6) (width 0.2) (layer "B.Cu") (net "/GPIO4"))
 (segment (start 148.59 91.44) (end 148.59 105.4) (width 0.2) (layer "B.Cu") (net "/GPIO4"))
 (segment (start 148.59 105.4) (end 143.9 105.4) (width 0.2) (layer "B.Cu") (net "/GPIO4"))
 (segment (start 170.82 75.6) (end 173.99 75.6) (width 0.2) (layer "B.Cu") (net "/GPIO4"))
 (segment (start 171 86) (end 147.485 86) (width 0.2) (layer "F.Cu") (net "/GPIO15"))
 (segment (start 171 80.5) (end 171 86) (width 0.2) (layer "F.Cu") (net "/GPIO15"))
 (segment (start 147.485 86) (end 147.485 106.895) (width 0.2) (layer "F.Cu") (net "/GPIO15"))
 (segment (start 147.485 106.895) (end 143.9 110.48) (width 0.2) (layer "F.Cu") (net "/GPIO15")))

